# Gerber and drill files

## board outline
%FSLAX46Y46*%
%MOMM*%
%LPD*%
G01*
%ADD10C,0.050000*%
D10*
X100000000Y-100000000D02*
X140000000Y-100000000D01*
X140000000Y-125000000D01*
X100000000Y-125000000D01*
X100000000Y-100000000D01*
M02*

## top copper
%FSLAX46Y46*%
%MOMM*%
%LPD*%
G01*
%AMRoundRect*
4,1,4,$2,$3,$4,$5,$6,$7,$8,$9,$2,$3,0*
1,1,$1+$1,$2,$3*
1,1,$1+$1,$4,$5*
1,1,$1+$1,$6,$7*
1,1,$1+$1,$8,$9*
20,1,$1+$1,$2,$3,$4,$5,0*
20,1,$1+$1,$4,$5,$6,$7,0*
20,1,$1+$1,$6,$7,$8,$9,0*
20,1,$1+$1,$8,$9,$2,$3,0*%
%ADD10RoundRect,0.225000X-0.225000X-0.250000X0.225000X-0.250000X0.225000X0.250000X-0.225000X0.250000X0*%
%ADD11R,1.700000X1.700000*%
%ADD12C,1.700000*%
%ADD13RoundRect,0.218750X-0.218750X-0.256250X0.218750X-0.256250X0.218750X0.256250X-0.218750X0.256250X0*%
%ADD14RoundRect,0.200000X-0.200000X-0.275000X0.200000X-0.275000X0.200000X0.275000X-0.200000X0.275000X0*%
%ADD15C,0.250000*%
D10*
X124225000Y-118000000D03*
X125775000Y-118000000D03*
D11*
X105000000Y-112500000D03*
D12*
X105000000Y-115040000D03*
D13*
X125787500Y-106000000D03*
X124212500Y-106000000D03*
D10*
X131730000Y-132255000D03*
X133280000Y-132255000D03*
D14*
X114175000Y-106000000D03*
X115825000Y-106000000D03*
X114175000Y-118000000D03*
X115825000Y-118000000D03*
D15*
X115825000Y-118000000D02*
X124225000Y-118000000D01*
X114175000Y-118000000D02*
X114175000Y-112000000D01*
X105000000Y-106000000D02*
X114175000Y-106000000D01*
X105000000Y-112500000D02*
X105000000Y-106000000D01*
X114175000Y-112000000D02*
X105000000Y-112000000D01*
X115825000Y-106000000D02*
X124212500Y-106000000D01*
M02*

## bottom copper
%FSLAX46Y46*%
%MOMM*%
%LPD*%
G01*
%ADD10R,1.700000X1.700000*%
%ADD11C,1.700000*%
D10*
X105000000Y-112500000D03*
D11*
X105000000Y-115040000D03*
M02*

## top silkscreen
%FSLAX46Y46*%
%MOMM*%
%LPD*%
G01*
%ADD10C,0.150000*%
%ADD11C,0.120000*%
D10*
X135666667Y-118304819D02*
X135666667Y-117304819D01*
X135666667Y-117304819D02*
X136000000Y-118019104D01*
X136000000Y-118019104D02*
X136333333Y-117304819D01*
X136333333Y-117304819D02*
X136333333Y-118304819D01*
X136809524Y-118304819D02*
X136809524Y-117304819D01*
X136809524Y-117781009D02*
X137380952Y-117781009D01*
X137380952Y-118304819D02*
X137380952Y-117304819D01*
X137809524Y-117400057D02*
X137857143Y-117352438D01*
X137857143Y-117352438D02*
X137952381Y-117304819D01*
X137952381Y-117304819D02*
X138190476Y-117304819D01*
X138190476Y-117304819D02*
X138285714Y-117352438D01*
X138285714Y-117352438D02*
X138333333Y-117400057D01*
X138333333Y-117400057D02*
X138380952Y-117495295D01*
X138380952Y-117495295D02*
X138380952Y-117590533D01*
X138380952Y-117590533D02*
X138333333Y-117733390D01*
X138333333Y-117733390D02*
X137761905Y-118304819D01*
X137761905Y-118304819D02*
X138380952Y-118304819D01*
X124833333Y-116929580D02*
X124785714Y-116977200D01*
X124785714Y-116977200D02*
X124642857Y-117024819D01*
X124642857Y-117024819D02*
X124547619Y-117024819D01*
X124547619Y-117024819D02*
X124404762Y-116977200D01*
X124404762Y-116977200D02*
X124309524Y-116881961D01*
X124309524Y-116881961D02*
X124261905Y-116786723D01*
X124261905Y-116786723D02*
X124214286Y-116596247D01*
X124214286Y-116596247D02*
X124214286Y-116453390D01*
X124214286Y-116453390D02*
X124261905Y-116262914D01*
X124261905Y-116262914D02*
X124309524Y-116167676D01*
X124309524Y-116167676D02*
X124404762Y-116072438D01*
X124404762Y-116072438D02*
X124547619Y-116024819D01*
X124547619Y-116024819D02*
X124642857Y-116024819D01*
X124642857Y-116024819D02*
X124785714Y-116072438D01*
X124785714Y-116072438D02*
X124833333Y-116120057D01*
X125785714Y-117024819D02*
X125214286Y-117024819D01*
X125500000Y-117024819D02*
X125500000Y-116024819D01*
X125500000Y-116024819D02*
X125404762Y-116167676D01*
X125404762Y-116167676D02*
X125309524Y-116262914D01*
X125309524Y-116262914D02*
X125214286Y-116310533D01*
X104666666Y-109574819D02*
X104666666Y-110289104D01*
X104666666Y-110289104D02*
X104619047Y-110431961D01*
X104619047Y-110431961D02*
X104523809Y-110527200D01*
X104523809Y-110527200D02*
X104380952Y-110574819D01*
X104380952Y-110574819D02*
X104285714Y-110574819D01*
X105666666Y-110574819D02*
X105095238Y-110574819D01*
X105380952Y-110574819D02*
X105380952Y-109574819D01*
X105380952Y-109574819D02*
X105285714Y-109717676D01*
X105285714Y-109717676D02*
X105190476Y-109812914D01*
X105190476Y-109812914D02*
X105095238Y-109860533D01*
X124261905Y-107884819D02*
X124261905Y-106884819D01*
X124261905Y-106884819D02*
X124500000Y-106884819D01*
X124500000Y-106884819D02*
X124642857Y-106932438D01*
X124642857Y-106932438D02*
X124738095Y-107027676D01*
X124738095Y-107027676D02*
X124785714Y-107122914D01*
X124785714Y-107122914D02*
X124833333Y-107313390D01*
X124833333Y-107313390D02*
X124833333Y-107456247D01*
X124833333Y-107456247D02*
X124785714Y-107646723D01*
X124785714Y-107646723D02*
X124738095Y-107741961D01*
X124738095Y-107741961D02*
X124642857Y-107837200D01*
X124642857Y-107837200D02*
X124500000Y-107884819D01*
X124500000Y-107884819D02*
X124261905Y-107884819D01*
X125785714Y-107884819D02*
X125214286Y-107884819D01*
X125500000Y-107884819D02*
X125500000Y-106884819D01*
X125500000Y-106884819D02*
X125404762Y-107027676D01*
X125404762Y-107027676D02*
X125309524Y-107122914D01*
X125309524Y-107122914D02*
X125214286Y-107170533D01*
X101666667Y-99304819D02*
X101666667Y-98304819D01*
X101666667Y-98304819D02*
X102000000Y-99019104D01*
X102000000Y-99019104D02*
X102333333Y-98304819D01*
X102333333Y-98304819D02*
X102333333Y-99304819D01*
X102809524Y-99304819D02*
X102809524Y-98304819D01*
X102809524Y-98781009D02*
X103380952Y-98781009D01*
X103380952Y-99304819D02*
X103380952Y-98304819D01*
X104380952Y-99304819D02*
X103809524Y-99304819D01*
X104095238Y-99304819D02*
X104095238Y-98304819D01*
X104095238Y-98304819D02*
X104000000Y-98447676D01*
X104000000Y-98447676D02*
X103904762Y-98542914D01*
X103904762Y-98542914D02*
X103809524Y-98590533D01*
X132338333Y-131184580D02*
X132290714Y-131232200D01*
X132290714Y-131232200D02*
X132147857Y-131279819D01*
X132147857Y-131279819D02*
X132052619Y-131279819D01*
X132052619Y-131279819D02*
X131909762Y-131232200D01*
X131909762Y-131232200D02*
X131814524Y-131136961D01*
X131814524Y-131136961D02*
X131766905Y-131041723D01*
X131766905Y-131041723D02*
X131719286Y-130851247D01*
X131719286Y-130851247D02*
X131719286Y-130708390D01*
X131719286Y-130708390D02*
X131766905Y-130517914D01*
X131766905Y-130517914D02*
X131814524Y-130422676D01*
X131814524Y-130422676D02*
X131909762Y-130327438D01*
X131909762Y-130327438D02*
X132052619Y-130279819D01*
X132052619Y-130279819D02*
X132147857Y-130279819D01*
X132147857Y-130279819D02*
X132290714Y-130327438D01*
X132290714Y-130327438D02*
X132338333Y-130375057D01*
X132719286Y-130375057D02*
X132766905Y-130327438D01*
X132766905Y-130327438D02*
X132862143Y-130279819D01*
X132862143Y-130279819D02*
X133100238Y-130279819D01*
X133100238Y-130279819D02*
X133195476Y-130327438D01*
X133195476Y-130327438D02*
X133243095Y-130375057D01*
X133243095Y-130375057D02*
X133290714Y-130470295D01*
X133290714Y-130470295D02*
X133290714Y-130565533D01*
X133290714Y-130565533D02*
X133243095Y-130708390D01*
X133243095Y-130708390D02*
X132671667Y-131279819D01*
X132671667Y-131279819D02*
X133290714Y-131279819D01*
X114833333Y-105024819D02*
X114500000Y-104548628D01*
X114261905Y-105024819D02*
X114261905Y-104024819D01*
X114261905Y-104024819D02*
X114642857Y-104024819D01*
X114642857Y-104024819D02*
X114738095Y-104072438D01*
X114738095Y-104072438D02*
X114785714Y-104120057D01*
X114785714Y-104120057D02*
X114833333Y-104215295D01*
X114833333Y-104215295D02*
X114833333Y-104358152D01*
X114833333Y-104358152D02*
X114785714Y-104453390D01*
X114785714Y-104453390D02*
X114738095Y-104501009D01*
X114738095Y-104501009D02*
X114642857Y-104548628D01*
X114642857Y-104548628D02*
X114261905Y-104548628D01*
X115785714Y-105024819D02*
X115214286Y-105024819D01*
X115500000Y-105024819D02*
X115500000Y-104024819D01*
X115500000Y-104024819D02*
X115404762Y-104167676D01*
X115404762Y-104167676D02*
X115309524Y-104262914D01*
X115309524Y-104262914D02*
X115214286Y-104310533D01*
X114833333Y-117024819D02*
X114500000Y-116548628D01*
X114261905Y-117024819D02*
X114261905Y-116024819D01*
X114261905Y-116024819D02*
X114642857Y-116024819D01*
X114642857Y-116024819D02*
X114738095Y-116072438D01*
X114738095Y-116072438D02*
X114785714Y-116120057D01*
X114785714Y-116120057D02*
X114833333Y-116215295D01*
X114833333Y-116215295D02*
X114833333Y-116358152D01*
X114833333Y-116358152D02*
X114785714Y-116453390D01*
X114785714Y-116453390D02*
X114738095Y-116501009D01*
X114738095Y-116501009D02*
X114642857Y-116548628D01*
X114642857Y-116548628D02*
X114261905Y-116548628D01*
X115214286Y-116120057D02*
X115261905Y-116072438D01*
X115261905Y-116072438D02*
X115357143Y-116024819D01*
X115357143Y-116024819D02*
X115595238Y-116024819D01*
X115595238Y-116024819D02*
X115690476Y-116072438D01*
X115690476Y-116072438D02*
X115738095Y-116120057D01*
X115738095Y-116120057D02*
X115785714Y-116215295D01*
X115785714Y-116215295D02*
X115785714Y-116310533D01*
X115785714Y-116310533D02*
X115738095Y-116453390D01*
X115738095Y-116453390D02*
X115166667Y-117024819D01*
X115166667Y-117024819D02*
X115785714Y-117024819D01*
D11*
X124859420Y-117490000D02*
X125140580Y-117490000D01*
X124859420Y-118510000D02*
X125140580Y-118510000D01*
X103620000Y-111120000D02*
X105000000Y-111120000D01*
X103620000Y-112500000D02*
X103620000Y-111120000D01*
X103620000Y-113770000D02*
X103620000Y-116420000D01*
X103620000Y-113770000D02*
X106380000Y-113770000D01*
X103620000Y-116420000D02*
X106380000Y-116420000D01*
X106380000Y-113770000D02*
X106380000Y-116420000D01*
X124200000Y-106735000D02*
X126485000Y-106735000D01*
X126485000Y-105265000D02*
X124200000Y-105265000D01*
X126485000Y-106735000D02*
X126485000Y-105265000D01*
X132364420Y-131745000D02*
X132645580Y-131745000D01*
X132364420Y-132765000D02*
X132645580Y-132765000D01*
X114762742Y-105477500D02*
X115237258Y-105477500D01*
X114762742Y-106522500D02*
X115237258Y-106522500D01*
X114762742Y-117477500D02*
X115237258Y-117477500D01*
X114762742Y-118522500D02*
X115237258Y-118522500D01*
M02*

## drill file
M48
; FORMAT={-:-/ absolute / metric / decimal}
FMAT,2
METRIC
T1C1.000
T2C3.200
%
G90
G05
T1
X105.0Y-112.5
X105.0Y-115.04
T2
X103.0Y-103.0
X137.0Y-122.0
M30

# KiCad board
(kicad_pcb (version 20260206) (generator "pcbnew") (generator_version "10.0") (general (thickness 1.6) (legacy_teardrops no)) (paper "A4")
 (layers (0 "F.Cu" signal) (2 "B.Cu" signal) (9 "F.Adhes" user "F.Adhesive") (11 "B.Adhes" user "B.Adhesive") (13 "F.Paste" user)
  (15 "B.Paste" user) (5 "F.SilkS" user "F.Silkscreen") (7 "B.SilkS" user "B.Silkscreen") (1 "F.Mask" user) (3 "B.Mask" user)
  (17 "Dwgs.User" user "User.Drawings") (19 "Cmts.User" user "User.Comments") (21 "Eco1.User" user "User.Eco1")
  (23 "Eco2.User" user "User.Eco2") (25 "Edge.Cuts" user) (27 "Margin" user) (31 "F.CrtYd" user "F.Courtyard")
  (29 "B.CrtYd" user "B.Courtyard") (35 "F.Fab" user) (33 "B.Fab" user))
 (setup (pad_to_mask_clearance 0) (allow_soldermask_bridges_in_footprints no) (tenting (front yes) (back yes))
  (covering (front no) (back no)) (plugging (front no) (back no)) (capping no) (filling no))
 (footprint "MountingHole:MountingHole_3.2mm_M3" (layer "F.Cu") (at 137 122)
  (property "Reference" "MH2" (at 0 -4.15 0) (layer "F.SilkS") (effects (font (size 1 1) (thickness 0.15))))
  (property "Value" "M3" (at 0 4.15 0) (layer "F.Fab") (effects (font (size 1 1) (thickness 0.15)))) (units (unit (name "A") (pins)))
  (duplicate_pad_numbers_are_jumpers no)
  (pad "" np_thru_hole circle (at 0 0) (size 3.2 3.2) (drill 3.2) (layers "*.Cu" "*.Mask")))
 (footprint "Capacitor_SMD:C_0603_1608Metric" (layer "F.Cu") (at 125 118)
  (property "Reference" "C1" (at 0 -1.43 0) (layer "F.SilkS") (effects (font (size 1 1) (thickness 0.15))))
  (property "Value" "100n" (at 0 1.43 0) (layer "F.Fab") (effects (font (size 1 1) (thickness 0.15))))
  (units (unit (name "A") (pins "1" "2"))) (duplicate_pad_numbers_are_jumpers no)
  (fp_line (start -0.14058 -0.51) (end 0.14058 -0.51) (stroke (width 0.12) (type solid)) (layer "F.SilkS"))
  (fp_line (start -0.14058 0.51) (end 0.14058 0.51) (stroke (width 0.12) (type solid)) (layer "F.SilkS"))
  (pad "1" smd roundrect (at -0.775 0) (size 0.9 0.95) (layers "F.Cu" "F.Mask" "F.Paste") (roundrect_rratio 0.25) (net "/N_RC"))
  (pad "2" smd roundrect (at 0.775 0) (size 0.9 0.95) (layers "F.Cu" "F.Mask" "F.Paste") (roundrect_rratio 0.25) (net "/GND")))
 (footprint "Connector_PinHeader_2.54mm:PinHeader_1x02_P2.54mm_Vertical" (layer "F.Cu") (at 105 112.5)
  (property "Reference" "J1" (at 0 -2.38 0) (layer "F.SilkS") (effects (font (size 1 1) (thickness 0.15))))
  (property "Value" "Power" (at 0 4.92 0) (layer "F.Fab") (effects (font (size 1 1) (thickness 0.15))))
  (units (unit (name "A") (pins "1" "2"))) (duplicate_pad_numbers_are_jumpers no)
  (fp_line (start -1.38 -1.38) (end 0 -1.38) (stroke (width 0.12) (type solid)) (layer "F.SilkS"))
  (fp_line (start -1.38 0) (end -1.38 -1.38) (stroke (width 0.12) (type solid)) (layer "F.SilkS"))
  (fp_line (start -1.38 1.27) (end -1.38 3.92) (stroke (width 0.12) (type solid)) (layer "F.SilkS"))
  (fp_line (start -1.38 1.27) (end 1.38 1.27) (stroke (width 0.12) (type solid)) (layer "F.SilkS"))
  (fp_line (start -1.38 3.92) (end 1.38 3.92) (stroke (width 0.12) (type solid)) (layer "F.SilkS"))
  (fp_line (start 1.38 1.27) (end 1.38 3.92) (stroke (width 0.12) (type solid)) (layer "F.SilkS"))
  (pad "1" thru_hole rect (at 0 0) (size 1.7 1.7) (drill 1) (layers "*.Cu" "*.Mask") (remove_unused_layers no) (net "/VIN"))
  (pad "2" thru_hole circle (at 0 2.54) (size 1.7 1.7) (drill 1) (layers "*.Cu" "*.Mask") (remove_unused_layers no) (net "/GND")))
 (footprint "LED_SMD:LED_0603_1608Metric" (layer "F.Cu") (at 125 106 180)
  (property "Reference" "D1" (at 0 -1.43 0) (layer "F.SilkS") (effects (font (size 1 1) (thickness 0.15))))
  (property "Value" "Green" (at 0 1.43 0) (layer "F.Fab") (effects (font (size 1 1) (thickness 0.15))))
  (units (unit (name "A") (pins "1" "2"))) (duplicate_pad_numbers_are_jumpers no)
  (fp_line (start 0.8 -0.735) (end -1.485 -0.735) (stroke (width 0.12) (type solid)) (layer "F.SilkS"))
  (fp_line (start -1.485 0.735) (end 0.8 0.735) (stroke (width 0.12) (type solid)) (layer "F.SilkS"))
  (fp_line (start -1.485 -0.735) (end -1.485 0.735) (stroke (width 0.12) (type solid)) (layer "F.SilkS"))
  (pad "1" smd roundrect (at -0.7875 0) (size 0.875 0.95) (layers "F.Cu" "F.Mask" "F.Paste") (roundrect_rratio 0.25) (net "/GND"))
  (pad "2" smd roundrect (at 0.7875 0) (size 0.875 0.95) (layers "F.Cu" "F.Mask" "F.Paste") (roundrect_rratio 0.25) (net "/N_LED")))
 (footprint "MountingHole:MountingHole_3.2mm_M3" (layer "F.Cu") (at 103 103)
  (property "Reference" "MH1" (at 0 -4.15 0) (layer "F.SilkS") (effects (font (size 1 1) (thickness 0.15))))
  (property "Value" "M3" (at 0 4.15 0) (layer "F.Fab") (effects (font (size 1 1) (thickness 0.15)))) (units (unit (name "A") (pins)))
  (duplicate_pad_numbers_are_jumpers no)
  (pad "" np_thru_hole circle (at 0 0) (size 3.2 3.2) (drill 3.2) (layers "*.Cu" "*.Mask")))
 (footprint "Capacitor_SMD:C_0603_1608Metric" (layer "F.Cu") (at 132.505 132.255)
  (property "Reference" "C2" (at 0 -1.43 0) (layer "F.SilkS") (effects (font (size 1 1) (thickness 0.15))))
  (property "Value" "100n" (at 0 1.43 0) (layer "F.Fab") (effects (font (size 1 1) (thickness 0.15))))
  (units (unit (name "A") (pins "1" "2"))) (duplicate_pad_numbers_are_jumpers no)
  (fp_line (start -0.14058 -0.51) (end 0.14058 -0.51) (stroke (width 0.12) (type solid)) (layer "F.SilkS"))
  (fp_line (start -0.14058 0.51) (end 0.14058 0.51) (stroke (width 0.12) (type solid)) (layer "F.SilkS"))
  (pad "1" smd roundrect (at -0.775 0) (size 0.9 0.95) (layers "F.Cu" "F.Mask" "F.Paste") (roundrect_rratio 0.25) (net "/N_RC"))
  (pad "2" smd roundrect (at 0.775 0) (size 0.9 0.95) (layers "F.Cu" "F.Mask" "F.Paste") (roundrect_rratio 0.25) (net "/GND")))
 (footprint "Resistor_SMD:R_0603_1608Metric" (layer "F.Cu") (at 115 106)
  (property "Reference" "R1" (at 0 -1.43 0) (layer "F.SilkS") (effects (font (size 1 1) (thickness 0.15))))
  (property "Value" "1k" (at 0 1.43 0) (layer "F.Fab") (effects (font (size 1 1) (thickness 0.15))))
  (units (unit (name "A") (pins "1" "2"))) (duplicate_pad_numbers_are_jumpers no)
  (fp_line (start -0.237258 -0.5225) (end 0.237258 -0.5225) (stroke (width 0.12) (type solid)) (layer "F.SilkS"))
  (fp_line (start -0.237258 0.5225) (end 0.237258 0.5225) (stroke (width 0.12) (type solid)) (layer "F.SilkS"))
  (pad "1" smd roundrect (at -0.825 0) (size 0.8 0.95) (layers "F.Cu" "F.Mask" "F.Paste") (roundrect_rratio 0.25) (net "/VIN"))
  (pad "2" smd roundrect (at 0.825 0) (size 0.8 0.95) (layers "F.Cu" "F.Mask" "F.Paste") (roundrect_rratio 0.25) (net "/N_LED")))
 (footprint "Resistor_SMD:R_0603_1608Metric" (layer "F.Cu") (at 115 118)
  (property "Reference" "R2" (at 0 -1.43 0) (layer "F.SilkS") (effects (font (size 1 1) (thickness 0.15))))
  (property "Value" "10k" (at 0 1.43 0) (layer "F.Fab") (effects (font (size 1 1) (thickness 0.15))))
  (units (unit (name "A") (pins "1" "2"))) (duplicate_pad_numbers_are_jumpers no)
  (fp_line (start -0.237258 -0.5225) (end 0.237258 -0.5225) (stroke (width 0.12) (type solid)) (layer "F.SilkS"))
  (fp_line (start -0.237258 0.5225) (end 0.237258 0.5225) (stroke (width 0.12) (type solid)) (layer "F.SilkS"))
  (pad "1" smd roundrect (at -0.825 0) (size 0.8 0.95) (layers "F.Cu" "F.Mask" "F.Paste") (roundrect_rratio 0.25) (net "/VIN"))
  (pad "2" smd roundrect (at 0.825 0) (size 0.8 0.95) (layers "F.Cu" "F.Mask" "F.Paste") (roundrect_rratio 0.25) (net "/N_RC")))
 (gr_rect (start 100 100) (end 140 125) (stroke (width 0.05) (type default)) (fill no) (layer "Edge.Cuts"))
 (segment (start 115.825 118) (end 124.225 118) (width 0.25) (layer "F.Cu") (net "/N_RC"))
 (segment (start 114.175 118) (end 114.175 112) (width 0.25) (layer "F.Cu") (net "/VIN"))
 (segment (start 105 106) (end 114.175 106) (width 0.25) (layer "F.Cu") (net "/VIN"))
 (segment (start 105 112.5) (end 105 106) (width 0.25) (layer "F.Cu") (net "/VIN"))
 (segment (start 114.175 112) (end 105 112) (width 0.25) (layer "F.Cu") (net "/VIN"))
 (segment (start 115.825 106) (end 124.2125 106) (width 0.25) (layer "F.Cu") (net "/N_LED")))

